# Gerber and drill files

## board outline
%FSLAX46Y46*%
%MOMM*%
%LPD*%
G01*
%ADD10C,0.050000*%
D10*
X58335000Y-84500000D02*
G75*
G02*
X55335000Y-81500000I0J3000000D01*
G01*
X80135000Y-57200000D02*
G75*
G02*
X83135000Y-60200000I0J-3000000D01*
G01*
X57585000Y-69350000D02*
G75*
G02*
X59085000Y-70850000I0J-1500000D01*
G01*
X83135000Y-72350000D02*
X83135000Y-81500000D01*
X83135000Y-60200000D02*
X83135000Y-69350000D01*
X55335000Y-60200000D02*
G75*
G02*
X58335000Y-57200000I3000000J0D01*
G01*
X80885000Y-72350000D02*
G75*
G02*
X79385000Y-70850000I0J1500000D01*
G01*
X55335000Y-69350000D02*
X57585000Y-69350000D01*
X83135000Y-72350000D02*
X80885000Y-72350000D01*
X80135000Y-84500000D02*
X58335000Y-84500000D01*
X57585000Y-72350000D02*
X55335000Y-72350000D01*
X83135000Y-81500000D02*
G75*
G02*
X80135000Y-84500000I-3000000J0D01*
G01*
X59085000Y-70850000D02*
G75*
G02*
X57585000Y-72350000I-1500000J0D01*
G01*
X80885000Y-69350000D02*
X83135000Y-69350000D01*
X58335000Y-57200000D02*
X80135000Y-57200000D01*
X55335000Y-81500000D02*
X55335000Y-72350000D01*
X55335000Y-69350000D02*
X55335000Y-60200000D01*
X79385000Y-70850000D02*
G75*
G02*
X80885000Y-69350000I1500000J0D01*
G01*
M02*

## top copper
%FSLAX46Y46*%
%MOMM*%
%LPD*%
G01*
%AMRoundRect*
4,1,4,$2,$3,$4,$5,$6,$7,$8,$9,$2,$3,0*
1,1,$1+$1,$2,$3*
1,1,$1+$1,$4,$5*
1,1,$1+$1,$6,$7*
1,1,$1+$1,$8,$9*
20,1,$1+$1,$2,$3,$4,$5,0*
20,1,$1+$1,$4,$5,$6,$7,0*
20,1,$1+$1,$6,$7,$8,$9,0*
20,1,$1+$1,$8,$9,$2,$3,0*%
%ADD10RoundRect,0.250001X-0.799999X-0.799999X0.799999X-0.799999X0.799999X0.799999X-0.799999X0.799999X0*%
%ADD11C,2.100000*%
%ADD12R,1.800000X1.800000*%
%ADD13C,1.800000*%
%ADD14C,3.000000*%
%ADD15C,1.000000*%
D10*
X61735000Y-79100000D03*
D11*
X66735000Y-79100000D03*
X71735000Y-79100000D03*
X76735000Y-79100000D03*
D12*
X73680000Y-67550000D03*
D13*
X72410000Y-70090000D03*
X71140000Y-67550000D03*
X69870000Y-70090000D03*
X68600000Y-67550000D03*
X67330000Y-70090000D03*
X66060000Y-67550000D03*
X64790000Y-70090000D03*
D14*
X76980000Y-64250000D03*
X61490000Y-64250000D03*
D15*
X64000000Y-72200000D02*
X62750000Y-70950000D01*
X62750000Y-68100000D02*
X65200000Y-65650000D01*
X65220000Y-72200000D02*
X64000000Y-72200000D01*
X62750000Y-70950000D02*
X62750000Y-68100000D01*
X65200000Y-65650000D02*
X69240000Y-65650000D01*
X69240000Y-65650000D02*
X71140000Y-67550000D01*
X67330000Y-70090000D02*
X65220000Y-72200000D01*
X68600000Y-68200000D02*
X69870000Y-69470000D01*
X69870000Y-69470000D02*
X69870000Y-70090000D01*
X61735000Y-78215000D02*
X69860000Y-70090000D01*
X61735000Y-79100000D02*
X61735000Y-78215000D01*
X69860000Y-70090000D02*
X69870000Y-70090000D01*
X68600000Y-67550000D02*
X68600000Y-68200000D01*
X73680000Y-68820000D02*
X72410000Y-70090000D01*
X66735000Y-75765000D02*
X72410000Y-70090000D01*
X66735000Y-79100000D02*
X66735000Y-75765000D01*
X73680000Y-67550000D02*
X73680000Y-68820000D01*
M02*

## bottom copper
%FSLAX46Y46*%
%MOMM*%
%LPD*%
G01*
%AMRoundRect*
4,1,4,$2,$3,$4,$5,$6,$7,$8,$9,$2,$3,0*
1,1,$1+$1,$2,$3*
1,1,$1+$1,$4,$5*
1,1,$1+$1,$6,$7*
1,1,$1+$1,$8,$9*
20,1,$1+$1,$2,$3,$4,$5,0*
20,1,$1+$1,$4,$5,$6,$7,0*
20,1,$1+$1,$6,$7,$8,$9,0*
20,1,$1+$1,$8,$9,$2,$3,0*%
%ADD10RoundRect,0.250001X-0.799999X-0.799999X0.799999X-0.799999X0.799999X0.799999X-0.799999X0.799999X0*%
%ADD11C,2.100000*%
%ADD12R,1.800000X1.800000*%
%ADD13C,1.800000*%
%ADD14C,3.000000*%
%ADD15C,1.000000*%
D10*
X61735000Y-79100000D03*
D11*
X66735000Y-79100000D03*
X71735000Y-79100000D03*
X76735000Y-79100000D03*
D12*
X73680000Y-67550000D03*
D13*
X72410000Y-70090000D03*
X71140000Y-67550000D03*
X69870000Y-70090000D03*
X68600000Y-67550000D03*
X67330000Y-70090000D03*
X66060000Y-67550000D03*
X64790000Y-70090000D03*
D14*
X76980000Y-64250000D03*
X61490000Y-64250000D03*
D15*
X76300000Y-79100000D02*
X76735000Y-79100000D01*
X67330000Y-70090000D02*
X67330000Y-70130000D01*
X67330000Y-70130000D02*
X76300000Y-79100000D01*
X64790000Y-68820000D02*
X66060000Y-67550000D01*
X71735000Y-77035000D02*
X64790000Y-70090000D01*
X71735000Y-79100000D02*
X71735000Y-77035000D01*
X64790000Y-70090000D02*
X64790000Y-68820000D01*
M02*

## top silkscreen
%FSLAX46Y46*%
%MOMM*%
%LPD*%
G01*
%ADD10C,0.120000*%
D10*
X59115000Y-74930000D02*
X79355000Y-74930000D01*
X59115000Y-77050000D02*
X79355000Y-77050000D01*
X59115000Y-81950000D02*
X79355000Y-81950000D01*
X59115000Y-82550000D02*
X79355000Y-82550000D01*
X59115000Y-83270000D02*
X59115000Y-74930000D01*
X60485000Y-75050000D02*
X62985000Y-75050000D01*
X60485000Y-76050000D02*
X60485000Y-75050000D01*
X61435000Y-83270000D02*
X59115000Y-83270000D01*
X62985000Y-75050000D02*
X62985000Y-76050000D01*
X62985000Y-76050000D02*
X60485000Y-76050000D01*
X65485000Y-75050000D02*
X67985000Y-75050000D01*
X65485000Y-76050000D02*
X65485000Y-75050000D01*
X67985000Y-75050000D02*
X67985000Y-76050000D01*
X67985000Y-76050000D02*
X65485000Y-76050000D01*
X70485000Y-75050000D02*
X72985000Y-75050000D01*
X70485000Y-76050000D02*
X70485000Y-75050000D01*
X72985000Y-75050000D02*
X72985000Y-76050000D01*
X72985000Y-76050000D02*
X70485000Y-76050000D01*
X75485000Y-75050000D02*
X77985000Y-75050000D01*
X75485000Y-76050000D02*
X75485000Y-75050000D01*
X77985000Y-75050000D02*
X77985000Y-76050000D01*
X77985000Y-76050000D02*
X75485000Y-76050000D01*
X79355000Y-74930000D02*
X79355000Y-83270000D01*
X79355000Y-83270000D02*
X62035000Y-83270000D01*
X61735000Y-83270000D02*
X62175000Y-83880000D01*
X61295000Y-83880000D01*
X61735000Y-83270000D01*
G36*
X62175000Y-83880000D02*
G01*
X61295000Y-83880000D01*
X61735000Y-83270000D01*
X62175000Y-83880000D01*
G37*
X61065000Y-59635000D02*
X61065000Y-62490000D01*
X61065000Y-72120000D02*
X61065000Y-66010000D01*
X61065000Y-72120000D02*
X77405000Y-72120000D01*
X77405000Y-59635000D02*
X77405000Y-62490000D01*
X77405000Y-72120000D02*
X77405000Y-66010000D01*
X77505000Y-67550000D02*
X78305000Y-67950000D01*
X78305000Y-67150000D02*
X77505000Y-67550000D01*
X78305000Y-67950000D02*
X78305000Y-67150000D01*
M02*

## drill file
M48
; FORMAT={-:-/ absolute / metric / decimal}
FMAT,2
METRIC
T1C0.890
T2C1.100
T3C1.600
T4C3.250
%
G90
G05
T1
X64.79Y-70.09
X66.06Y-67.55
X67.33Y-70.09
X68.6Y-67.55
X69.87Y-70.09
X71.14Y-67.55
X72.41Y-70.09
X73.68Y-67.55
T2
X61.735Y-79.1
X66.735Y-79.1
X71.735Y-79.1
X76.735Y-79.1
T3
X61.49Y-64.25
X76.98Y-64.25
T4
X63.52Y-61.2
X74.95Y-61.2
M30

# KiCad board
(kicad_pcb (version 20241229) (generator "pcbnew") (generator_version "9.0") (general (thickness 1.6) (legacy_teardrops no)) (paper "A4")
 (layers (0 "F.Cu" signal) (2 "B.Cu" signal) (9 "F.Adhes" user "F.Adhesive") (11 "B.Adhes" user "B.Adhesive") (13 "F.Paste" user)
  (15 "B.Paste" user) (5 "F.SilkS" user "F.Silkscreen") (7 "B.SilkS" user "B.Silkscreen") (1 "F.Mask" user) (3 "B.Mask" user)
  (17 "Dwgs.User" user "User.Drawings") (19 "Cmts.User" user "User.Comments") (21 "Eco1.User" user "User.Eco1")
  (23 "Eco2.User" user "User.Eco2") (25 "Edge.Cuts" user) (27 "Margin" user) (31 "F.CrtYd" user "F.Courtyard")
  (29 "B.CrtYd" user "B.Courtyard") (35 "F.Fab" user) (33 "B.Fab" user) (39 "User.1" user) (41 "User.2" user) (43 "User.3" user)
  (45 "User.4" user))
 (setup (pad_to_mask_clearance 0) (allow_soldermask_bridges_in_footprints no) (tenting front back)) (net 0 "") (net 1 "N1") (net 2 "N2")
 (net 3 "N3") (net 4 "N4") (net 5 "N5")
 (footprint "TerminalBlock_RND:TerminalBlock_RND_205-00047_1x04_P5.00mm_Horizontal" (layer "F.Cu") (at 61.735 79.1)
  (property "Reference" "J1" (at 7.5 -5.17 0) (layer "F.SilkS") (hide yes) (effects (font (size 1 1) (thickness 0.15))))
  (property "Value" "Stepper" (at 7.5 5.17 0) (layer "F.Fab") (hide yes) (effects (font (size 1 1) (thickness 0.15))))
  (fp_line (start -2.62 -4.17) (end 17.62 -4.17) (stroke (width 0.12) (type solid)) (layer "F.SilkS"))
  (fp_line (start -2.62 -2.05) (end 17.62 -2.05) (stroke (width 0.12) (type solid)) (layer "F.SilkS"))
  (fp_line (start -2.62 2.85) (end 17.62 2.85) (stroke (width 0.12) (type solid)) (layer "F.SilkS"))
  (fp_line (start -2.62 3.45) (end 17.62 3.45) (stroke (width 0.12) (type solid)) (layer "F.SilkS"))
  (fp_line (start -2.62 4.17) (end -2.62 -4.17) (stroke (width 0.12) (type solid)) (layer "F.SilkS"))
  (fp_line (start -1.25 -4.05) (end 1.25 -4.05) (stroke (width 0.12) (type solid)) (layer "F.SilkS"))
  (fp_line (start -1.25 -3.05) (end -1.25 -4.05) (stroke (width 0.12) (type solid)) (layer "F.SilkS"))
  (fp_line (start -0.3 4.17) (end -2.62 4.17) (stroke (width 0.12) (type solid)) (layer "F.SilkS"))
  (fp_line (start 1.25 -4.05) (end 1.25 -3.05) (stroke (width 0.12) (type solid)) (layer "F.SilkS"))
  (fp_line (start 1.25 -3.05) (end -1.25 -3.05) (stroke (width 0.12) (type solid)) (layer "F.SilkS"))
  (fp_line (start 3.75 -4.05) (end 6.25 -4.05) (stroke (width 0.12) (type solid)) (layer "F.SilkS"))
  (fp_line (start 3.75 -3.05) (end 3.75 -4.05) (stroke (width 0.12) (type solid)) (layer "F.SilkS"))
  (fp_line (start 6.25 -4.05) (end 6.25 -3.05) (stroke (width 0.12) (type solid)) (layer "F.SilkS"))
  (fp_line (start 6.25 -3.05) (end 3.75 -3.05) (stroke (width 0.12) (type solid)) (layer "F.SilkS"))
  (fp_line (start 8.75 -4.05) (end 11.25 -4.05) (stroke (width 0.12) (type solid)) (layer "F.SilkS"))
  (fp_line (start 8.75 -3.05) (end 8.75 -4.05) (stroke (width 0.12) (type solid)) (layer "F.SilkS"))
  (fp_line (start 11.25 -4.05) (end 11.25 -3.05) (stroke (width 0.12) (type solid)) (layer "F.SilkS"))
  (fp_line (start 11.25 -3.05) (end 8.75 -3.05) (stroke (width 0.12) (type solid)) (layer "F.SilkS"))
  (fp_line (start 13.75 -4.05) (end 16.25 -4.05) (stroke (width 0.12) (type solid)) (layer "F.SilkS"))
  (fp_line (start 13.75 -3.05) (end 13.75 -4.05) (stroke (width 0.12) (type solid)) (layer "F.SilkS"))
  (fp_line (start 16.25 -4.05) (end 16.25 -3.05) (stroke (width 0.12) (type solid)) (layer "F.SilkS"))
  (fp_line (start 16.25 -3.05) (end 13.75 -3.05) (stroke (width 0.12) (type solid)) (layer "F.SilkS"))
  (fp_line (start 17.62 -4.17) (end 17.62 4.17) (stroke (width 0.12) (type solid)) (layer "F.SilkS"))
  (fp_line (start 17.62 4.17) (end 0.3 4.17) (stroke (width 0.12) (type solid)) (layer "F.SilkS"))
  (fp_poly (pts (xy 0 4.17) (xy 0.44 4.78) (xy -0.44 4.78)) (stroke (width 0.12) (type solid)) (fill yes) (layer "F.SilkS"))
  (pad "1" thru_hole roundrect (at 0 0) (size 2.1 2.1) (drill 1.1) (layers "*.Cu" "*.Mask") (remove_unused_layers no)
   (roundrect_rratio 0.119048) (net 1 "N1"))
  (pad "2" thru_hole circle (at 5 0) (size 2.1 2.1) (drill 1.1) (layers "*.Cu" "*.Mask") (remove_unused_layers no) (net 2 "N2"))
  (pad "3" thru_hole circle (at 10 0) (size 2.1 2.1) (drill 1.1) (layers "*.Cu" "*.Mask") (remove_unused_layers no) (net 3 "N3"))
  (pad "4" thru_hole circle (at 15 0) (size 2.1 2.1) (drill 1.1) (layers "*.Cu" "*.Mask") (remove_unused_layers no) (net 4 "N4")))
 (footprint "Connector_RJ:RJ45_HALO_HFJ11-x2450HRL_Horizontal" (layer "F.Cu") (at 73.68 67.55 180)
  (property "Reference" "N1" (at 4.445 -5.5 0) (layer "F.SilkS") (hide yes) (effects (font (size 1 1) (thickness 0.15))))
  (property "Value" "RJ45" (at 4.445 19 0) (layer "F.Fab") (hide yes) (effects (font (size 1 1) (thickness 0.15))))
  (fp_line (start 12.615 7.915) (end 12.615 5.06) (stroke (width 0.12) (type solid)) (layer "F.SilkS"))
  (fp_line (start 12.615 -4.57) (end 12.615 1.54) (stroke (width 0.12) (type solid)) (layer "F.SilkS"))
  (fp_line (start 12.615 -4.57) (end -3.725 -4.57) (stroke (width 0.12) (type solid)) (layer "F.SilkS"))
  (fp_line (start -3.725 7.915) (end -3.725 5.06) (stroke (width 0.12) (type solid)) (layer "F.SilkS"))
  (fp_line (start -3.725 -4.57) (end -3.725 1.54) (stroke (width 0.12) (type solid)) (layer "F.SilkS"))
  (fp_line (start -3.825 0) (end -4.625 -0.4) (stroke (width 0.12) (type solid)) (layer "F.SilkS"))
  (fp_line (start -4.625 0.4) (end -3.825 0) (stroke (width 0.12) (type solid)) (layer "F.SilkS"))
  (fp_line (start -4.625 -0.4) (end -4.625 0.4) (stroke (width 0.12) (type solid)) (layer "F.SilkS"))
  (pad "" np_thru_hole circle (at -1.27 6.35 180) (size 3.25 3.25) (drill 3.25) (layers "*.Cu" "*.Mask"))
  (pad "" np_thru_hole circle (at 10.16 6.35 180) (size 3.25 3.25) (drill 3.25) (layers "*.Cu" "*.Mask"))
  (pad "1" thru_hole rect (at 0 0 180) (size 1.8 1.8) (drill 0.89) (layers "*.Cu" "*.Mask") (remove_unused_layers no) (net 2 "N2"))
  (pad "2" thru_hole circle (at 1.27 -2.54 180) (size 1.8 1.8) (drill 0.89) (layers "*.Cu" "*.Mask") (remove_unused_layers no) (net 2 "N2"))
  (pad "3" thru_hole circle (at 2.54 0 180) (size 1.8 1.8) (drill 0.89) (layers "*.Cu" "*.Mask") (remove_unused_layers no) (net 4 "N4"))
  (pad "4" thru_hole circle (at 3.81 -2.54 180) (size 1.8 1.8) (drill 0.89) (layers "*.Cu" "*.Mask") (remove_unused_layers no) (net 1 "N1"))
  (pad "5" thru_hole circle (at 5.08 0 180) (size 1.8 1.8) (drill 0.89) (layers "*.Cu" "*.Mask") (remove_unused_layers no) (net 1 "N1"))
  (pad "6" thru_hole circle (at 6.35 -2.54 180) (size 1.8 1.8) (drill 0.89) (layers "*.Cu" "*.Mask") (remove_unused_layers no) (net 4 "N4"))
  (pad "7" thru_hole circle (at 7.62 0 180) (size 1.8 1.8) (drill 0.89) (layers "*.Cu" "*.Mask") (remove_unused_layers no) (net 3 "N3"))
  (pad "8" thru_hole circle (at 8.89 -2.54 180) (size 1.8 1.8) (drill 0.89) (layers "*.Cu" "*.Mask") (remove_unused_layers no) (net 3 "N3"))
  (pad "SH" thru_hole circle (at -3.3 3.3 180) (size 3 3) (drill 1.6) (layers "*.Cu" "*.Mask") (remove_unused_layers no) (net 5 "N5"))
  (pad "SH" thru_hole circle (at 12.19 3.3 180) (size 3 3) (drill 1.6) (layers "*.Cu" "*.Mask") (remove_unused_layers no) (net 5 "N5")))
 (gr_arc (start 58.335 84.5) (mid 56.21368 83.62132) (end 55.335 81.5) (stroke (width 0.05) (type default)) (layer "Edge.Cuts"))
 (gr_arc (start 80.135 57.2) (mid 82.25632 58.07868) (end 83.135 60.2) (stroke (width 0.05) (type default)) (layer "Edge.Cuts"))
 (gr_arc (start 57.585 69.35) (mid 58.64566 69.78934) (end 59.085 70.85) (stroke (width 0.05) (type default)) (layer "Edge.Cuts"))
 (gr_line (start 83.135 72.35) (end 83.135 81.5) (stroke (width 0.05) (type default)) (layer "Edge.Cuts"))
 (gr_line (start 83.135 60.2) (end 83.135 69.35) (stroke (width 0.05) (type default)) (layer "Edge.Cuts"))
 (gr_arc (start 55.335 60.2) (mid 56.21368 58.07868) (end 58.335 57.2) (stroke (width 0.05) (type default)) (layer "Edge.Cuts"))
 (gr_arc (start 80.885 72.35) (mid 79.82434 71.91066) (end 79.385 70.85) (stroke (width 0.05) (type default)) (layer "Edge.Cuts"))
 (gr_line (start 55.335 69.35) (end 57.585 69.35) (stroke (width 0.05) (type solid)) (layer "Edge.Cuts"))
 (gr_line (start 83.135 72.35) (end 80.885 72.35) (stroke (width 0.05) (type solid)) (layer "Edge.Cuts"))
 (gr_line (start 80.135 84.5) (end 58.335 84.5) (stroke (width 0.05) (type default)) (layer "Edge.Cuts"))
 (gr_line (start 57.585 72.35) (end 55.335 72.35) (stroke (width 0.05) (type solid)) (layer "Edge.Cuts"))
 (gr_arc (start 83.135 81.5) (mid 82.25632 83.62132) (end 80.135 84.5) (stroke (width 0.05) (type default)) (layer "Edge.Cuts"))
 (gr_arc (start 59.085 70.85) (mid 58.64566 71.91066) (end 57.585 72.35) (stroke (width 0.05) (type default)) (layer "Edge.Cuts"))
 (gr_line (start 80.885 69.35) (end 83.135 69.35) (stroke (width 0.05) (type solid)) (layer "Edge.Cuts"))
 (gr_line (start 58.335 57.2) (end 80.135 57.2) (stroke (width 0.05) (type default)) (layer "Edge.Cuts"))
 (gr_line (start 55.335 81.5) (end 55.335 72.35) (stroke (width 0.05) (type default)) (layer "Edge.Cuts"))
 (gr_line (start 55.335 69.35) (end 55.335 60.2) (stroke (width 0.05) (type default)) (layer "Edge.Cuts"))
 (gr_arc (start 79.385 70.85) (mid 79.82434 69.78934) (end 80.885 69.35) (stroke (width 0.05) (type default)) (layer "Edge.Cuts"))
 (segment (start 64 72.2) (end 62.75 70.95) (width 1) (layer "F.Cu") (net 4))
 (segment (start 62.75 68.1) (end 65.2 65.65) (width 1) (layer "F.Cu") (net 4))
 (segment (start 65.22 72.2) (end 64 72.2) (width 1) (layer "F.Cu") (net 4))
 (segment (start 62.75 70.95) (end 62.75 68.1) (width 1) (layer "F.Cu") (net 4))
 (segment (start 65.2 65.65) (end 69.24 65.65) (width 1) (layer "F.Cu") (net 4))
 (segment (start 69.24 65.65) (end 71.14 67.55) (width 1) (layer "F.Cu") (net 4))
 (segment (start 67.33 70.09) (end 65.22 72.2) (width 1) (layer "F.Cu") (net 4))
 (segment (start 76.3 79.1) (end 76.735 79.1) (width 1) (layer "B.Cu") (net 4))
 (segment (start 67.33 70.09) (end 67.33 70.13) (width 1) (layer "B.Cu") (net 4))
 (segment (start 67.33 70.13) (end 76.3 79.1) (width 1) (layer "B.Cu") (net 4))
 (segment (start 64.79 68.82) (end 66.06 67.55) (width 1) (layer "B.Cu") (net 3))
 (segment (start 71.735 77.035) (end 64.79 70.09) (width 1) (layer "B.Cu") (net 3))
 (segment (start 71.735 79.1) (end 71.735 77.035) (width 1) (layer "B.Cu") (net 3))
 (segment (start 64.79 70.09) (end 64.79 68.82) (width 1) (layer "B.Cu") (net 3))
 (segment (start 68.6 68.2) (end 69.87 69.47) (width 1) (layer "F.Cu") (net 1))
 (segment (start 69.87 69.47) (end 69.87 70.09) (width 1) (layer "F.Cu") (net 1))
 (segment (start 61.735 78.215) (end 69.86 70.09) (width 1) (layer "F.Cu") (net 1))
 (segment (start 61.735 79.1) (end 61.735 78.215) (width 1) (layer "F.Cu") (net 1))
 (segment (start 69.86 70.09) (end 69.87 70.09) (width 1) (layer "F.Cu") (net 1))
 (segment (start 68.6 67.55) (end 68.6 68.2) (width 1) (layer "F.Cu") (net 1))
 (segment (start 73.68 68.82) (end 72.41 70.09) (width 1) (layer "F.Cu") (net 2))
 (segment (start 66.735 75.765) (end 72.41 70.09) (width 1) (layer "F.Cu") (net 2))
 (segment (start 66.735 79.1) (end 66.735 75.765) (width 1) (layer "F.Cu") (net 2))
 (segment (start 73.68 67.55) (end 73.68 68.82) (width 1) (layer "F.Cu") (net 2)))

